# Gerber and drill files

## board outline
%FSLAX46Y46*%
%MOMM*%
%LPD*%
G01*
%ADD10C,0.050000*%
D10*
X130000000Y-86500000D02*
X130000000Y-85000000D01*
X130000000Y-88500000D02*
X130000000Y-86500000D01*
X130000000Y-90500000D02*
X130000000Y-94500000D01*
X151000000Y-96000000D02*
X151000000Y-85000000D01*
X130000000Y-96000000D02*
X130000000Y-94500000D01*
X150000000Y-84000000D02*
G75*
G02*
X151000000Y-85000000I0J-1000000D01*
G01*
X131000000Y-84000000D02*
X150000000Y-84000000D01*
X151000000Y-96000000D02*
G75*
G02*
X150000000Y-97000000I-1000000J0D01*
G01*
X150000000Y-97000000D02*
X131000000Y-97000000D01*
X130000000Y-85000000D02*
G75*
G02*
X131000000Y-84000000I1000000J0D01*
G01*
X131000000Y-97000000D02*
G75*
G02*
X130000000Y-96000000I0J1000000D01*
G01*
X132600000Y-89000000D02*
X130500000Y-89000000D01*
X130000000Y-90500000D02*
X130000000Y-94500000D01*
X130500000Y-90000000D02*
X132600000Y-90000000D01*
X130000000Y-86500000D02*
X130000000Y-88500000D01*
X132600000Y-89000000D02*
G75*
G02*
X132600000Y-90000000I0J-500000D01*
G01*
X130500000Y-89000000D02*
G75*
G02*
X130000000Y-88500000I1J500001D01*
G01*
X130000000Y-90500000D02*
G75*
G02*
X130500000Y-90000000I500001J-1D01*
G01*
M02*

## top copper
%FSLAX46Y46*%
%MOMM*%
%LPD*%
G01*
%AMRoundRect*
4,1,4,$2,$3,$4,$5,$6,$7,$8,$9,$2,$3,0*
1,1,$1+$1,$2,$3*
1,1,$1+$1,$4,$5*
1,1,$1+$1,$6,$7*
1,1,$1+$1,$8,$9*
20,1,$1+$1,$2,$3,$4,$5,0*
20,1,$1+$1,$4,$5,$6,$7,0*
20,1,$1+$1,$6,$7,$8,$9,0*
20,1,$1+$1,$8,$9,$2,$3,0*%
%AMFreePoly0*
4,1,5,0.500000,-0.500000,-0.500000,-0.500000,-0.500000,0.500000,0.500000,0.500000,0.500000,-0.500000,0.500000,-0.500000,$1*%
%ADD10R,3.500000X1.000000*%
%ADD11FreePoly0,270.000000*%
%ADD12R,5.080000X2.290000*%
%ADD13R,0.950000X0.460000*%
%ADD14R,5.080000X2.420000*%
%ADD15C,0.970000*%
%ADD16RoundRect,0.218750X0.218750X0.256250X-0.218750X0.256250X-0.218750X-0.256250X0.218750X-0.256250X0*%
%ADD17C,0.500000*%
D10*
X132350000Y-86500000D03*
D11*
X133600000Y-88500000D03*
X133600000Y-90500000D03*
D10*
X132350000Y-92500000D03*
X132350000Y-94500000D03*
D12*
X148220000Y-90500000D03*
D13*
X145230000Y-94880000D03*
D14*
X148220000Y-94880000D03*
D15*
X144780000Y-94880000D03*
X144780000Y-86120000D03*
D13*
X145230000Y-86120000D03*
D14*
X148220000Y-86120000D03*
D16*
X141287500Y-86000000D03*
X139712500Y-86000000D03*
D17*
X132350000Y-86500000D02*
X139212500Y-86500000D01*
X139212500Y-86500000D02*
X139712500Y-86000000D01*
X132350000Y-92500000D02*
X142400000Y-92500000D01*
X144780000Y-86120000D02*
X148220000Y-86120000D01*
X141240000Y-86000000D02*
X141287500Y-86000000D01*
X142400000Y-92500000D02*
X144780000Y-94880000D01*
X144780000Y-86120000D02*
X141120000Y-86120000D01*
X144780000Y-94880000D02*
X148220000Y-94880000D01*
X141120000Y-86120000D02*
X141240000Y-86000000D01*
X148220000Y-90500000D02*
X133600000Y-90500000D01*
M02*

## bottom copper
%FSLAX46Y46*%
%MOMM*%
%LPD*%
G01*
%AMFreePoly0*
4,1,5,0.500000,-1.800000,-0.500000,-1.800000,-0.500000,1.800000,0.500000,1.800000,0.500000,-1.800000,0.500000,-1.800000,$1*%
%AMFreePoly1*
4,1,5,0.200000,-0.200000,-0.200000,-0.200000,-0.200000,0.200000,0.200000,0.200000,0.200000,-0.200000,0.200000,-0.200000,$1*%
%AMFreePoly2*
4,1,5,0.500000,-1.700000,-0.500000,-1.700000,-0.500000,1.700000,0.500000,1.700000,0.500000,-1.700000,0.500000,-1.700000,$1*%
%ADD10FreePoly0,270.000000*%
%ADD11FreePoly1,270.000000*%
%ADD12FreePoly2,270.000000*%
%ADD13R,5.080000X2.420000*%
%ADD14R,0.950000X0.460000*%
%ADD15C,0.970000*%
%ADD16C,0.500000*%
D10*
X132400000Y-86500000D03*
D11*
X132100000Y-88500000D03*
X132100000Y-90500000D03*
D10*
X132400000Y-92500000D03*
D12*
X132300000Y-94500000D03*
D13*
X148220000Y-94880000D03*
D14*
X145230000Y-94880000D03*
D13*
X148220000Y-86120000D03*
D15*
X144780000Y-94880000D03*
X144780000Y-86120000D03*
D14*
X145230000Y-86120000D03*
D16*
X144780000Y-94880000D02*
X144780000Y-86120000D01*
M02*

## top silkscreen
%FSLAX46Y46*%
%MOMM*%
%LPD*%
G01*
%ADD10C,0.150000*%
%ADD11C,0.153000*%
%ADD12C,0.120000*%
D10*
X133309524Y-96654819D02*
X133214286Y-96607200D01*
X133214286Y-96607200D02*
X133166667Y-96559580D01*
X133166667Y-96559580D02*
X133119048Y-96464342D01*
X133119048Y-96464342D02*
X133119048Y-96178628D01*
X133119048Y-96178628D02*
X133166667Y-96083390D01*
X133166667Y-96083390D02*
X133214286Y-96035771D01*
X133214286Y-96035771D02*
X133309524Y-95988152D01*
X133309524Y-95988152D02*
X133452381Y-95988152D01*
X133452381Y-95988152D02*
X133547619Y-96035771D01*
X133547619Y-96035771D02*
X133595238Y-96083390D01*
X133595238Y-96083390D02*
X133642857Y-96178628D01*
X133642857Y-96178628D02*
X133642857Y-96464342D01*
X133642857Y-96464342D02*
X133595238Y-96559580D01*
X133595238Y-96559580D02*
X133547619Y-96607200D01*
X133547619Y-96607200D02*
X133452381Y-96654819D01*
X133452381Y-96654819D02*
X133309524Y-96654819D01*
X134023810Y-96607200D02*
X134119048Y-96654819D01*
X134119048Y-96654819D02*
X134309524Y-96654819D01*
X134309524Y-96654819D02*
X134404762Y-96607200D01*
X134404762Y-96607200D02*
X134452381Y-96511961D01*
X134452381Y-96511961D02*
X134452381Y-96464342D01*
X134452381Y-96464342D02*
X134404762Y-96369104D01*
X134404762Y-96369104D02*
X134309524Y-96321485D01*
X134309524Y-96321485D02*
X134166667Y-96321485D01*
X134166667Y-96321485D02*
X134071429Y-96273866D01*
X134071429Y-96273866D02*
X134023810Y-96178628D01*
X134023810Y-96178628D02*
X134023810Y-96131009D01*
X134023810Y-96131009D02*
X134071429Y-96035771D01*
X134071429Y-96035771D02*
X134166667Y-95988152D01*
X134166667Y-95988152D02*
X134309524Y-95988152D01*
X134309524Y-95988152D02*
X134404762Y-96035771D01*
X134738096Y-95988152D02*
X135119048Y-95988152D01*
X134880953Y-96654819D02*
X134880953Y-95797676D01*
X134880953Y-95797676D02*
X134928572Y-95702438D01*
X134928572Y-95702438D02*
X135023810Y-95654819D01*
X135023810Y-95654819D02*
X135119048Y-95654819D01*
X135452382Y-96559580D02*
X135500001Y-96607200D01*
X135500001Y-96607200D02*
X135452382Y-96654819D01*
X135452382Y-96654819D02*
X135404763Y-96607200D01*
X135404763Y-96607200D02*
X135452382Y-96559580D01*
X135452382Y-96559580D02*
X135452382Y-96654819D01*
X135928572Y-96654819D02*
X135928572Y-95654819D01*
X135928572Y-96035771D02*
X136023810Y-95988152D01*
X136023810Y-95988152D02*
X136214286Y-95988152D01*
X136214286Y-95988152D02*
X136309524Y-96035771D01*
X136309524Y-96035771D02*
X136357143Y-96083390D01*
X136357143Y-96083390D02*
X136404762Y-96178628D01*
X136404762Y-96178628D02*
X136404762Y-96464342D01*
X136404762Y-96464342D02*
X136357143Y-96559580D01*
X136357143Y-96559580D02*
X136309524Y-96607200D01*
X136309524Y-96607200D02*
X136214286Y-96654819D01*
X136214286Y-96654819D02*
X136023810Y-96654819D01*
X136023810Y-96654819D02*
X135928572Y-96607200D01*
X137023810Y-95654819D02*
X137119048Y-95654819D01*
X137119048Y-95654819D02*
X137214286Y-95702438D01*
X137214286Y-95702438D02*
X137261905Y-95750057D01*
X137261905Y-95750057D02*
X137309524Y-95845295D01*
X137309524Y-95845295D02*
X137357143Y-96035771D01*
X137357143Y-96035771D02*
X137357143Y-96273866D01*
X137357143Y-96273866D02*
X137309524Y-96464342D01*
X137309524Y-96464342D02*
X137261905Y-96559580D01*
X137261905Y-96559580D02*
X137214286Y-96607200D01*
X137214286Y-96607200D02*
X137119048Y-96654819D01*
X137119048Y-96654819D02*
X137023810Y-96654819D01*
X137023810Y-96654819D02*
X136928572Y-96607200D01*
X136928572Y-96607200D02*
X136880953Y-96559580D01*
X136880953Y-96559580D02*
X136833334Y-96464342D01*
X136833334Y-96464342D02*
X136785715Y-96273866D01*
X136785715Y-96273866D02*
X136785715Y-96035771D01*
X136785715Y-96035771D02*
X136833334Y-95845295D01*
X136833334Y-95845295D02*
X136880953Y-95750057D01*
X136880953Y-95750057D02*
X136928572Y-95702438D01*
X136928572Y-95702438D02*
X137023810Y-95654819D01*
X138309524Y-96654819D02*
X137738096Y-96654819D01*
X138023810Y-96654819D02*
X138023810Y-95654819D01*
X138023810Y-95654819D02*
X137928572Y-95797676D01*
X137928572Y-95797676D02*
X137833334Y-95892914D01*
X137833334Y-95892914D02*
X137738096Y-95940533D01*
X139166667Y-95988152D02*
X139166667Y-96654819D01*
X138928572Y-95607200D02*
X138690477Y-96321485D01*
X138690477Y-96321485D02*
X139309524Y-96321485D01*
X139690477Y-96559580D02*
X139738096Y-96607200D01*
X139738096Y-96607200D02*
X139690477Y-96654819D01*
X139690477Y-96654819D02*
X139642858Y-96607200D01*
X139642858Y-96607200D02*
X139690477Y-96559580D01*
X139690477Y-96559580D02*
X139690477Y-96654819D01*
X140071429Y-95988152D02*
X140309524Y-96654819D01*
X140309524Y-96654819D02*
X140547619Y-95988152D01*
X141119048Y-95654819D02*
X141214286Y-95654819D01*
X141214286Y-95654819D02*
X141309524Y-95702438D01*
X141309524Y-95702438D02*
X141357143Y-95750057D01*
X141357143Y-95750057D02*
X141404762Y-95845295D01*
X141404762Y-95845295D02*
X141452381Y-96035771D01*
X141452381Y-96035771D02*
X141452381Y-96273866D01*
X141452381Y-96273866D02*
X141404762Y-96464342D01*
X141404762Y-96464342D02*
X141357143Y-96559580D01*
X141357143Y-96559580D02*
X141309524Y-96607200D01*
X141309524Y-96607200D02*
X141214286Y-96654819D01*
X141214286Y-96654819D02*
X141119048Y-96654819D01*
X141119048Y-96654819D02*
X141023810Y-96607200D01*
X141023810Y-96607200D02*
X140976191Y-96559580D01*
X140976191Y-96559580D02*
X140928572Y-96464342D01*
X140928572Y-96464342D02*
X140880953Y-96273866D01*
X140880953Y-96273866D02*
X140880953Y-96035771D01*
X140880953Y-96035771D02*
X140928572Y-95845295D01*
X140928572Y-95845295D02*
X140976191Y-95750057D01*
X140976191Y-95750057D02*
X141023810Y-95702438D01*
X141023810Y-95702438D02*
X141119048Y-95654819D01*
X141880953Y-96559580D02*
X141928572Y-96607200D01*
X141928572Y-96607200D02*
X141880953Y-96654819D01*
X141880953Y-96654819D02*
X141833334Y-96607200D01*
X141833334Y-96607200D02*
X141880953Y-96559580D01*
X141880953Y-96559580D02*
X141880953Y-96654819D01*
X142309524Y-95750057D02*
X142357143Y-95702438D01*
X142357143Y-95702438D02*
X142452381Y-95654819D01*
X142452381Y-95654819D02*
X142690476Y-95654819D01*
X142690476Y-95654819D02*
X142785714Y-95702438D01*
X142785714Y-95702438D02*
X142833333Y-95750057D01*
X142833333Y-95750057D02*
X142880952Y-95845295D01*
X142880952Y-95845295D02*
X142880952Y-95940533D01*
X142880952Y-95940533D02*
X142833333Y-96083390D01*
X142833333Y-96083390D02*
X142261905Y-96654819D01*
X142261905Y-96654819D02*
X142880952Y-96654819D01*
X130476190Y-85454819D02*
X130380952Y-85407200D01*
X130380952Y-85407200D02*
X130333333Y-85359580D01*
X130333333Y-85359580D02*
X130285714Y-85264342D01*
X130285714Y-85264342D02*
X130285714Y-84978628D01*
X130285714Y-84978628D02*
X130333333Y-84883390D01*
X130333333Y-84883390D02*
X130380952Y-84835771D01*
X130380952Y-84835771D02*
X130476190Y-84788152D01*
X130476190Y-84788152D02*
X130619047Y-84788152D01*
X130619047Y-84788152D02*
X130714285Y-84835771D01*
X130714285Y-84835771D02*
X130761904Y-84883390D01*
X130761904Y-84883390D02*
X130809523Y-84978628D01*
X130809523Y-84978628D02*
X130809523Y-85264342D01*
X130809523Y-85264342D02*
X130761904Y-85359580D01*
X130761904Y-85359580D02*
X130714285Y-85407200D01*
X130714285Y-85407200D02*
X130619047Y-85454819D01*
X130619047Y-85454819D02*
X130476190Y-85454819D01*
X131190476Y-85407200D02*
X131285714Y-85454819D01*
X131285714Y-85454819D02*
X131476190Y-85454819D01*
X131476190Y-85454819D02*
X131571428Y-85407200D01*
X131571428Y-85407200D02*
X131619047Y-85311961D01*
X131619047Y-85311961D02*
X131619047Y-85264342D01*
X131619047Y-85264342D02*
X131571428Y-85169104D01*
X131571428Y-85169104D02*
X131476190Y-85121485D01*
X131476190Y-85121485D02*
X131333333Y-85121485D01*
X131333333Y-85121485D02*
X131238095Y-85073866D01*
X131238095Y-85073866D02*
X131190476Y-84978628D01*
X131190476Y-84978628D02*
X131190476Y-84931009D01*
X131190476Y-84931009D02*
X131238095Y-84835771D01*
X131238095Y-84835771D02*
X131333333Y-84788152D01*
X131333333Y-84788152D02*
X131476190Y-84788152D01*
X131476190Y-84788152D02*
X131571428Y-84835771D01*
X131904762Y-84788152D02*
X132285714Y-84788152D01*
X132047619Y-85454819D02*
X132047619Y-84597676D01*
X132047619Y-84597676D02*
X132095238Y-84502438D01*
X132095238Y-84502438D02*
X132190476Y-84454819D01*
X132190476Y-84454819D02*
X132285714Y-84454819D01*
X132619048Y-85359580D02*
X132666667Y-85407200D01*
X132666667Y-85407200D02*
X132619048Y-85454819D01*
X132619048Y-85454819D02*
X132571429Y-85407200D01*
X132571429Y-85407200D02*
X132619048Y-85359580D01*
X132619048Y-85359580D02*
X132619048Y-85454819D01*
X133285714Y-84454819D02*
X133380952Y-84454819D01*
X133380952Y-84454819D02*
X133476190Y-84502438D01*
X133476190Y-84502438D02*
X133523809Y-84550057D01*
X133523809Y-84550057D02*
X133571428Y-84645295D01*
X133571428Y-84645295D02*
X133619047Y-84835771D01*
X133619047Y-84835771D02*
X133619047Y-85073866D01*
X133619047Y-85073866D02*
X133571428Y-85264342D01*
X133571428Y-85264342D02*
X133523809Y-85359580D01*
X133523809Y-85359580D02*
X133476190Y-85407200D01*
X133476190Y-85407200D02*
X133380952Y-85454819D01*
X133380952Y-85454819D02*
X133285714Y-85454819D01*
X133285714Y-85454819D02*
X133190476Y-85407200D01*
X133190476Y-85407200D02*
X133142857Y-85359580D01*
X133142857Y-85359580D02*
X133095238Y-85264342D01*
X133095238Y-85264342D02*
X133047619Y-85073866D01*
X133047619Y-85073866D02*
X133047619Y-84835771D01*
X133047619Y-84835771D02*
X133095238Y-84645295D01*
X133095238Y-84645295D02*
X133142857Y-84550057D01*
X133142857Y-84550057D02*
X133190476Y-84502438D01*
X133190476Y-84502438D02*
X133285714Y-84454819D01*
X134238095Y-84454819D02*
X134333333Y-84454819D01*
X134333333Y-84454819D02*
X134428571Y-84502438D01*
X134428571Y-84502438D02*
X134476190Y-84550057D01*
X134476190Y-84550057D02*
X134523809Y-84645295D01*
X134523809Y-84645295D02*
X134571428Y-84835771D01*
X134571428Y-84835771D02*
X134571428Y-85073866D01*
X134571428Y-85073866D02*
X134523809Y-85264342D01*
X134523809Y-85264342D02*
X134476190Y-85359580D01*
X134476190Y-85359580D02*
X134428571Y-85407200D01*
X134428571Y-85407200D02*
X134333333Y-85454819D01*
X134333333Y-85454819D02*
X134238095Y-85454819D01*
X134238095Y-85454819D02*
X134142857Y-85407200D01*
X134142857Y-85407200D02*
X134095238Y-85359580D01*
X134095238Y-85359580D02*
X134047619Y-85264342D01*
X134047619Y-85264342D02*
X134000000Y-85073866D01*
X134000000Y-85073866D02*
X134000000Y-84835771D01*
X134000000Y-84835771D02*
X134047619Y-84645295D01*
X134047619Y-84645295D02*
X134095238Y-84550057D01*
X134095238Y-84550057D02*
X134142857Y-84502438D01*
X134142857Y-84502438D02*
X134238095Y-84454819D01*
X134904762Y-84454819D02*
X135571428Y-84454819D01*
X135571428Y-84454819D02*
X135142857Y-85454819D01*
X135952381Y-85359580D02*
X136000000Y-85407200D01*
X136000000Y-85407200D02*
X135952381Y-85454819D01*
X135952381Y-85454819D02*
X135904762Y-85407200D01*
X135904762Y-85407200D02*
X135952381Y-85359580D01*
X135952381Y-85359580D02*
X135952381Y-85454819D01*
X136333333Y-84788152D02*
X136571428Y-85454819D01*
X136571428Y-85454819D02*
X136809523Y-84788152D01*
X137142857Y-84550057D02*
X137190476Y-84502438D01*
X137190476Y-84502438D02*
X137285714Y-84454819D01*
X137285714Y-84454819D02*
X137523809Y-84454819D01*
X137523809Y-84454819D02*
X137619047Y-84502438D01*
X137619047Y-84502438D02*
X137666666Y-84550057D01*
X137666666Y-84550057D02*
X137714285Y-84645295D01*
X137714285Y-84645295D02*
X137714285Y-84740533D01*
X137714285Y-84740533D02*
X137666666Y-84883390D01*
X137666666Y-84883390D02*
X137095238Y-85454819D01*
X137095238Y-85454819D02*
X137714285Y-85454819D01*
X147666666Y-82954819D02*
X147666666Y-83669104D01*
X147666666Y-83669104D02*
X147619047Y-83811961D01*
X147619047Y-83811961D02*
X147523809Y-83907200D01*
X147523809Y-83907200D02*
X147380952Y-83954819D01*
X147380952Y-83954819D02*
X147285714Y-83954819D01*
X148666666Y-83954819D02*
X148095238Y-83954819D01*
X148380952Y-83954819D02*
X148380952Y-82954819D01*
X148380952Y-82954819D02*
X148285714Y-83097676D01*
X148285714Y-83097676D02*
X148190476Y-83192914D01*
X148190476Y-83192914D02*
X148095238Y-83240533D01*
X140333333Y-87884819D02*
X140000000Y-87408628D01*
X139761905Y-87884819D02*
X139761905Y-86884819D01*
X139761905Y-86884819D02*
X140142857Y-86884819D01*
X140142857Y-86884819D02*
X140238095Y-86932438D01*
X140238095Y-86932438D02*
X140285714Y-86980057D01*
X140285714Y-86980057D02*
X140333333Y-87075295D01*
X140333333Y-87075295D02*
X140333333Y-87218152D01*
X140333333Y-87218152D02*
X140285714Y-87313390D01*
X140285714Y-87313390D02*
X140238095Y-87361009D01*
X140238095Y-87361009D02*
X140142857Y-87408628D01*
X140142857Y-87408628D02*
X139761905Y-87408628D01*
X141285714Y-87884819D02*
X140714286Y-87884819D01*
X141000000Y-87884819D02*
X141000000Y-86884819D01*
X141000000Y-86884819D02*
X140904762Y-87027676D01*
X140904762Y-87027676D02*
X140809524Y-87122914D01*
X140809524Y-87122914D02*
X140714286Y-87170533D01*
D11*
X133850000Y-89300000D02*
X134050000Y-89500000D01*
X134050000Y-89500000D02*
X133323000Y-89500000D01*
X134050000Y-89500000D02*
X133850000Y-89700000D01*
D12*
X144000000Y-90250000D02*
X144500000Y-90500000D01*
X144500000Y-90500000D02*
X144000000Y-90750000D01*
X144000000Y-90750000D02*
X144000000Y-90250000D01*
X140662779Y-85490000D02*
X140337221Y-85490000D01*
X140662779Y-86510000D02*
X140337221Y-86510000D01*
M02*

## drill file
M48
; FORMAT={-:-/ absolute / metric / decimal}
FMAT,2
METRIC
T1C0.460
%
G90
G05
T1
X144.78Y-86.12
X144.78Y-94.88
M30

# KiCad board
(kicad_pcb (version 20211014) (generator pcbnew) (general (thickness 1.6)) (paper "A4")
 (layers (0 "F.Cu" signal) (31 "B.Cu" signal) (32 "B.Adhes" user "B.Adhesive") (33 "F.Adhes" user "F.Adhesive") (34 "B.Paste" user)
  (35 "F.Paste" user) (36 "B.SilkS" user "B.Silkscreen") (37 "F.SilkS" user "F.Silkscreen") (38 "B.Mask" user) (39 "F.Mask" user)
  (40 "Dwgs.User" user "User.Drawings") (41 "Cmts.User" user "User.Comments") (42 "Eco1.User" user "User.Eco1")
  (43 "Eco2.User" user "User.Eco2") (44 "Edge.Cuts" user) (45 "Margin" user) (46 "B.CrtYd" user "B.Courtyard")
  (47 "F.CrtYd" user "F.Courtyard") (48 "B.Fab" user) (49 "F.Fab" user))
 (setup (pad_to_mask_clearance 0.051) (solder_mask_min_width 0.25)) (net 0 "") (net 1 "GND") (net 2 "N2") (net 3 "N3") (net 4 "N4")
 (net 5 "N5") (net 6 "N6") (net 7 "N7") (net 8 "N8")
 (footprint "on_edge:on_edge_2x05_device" (layer "F.Cu") (at 130 90.5 -90)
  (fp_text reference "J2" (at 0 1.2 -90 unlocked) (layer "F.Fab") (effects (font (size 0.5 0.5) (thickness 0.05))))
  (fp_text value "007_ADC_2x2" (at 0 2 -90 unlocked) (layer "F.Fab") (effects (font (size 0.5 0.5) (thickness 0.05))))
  (fp_line (start -1.2 -3.85) (end -1 -4.05) (layer "F.SilkS") (width 0.153))
  (fp_line (start -1 -4.05) (end -1 -3.323) (layer "F.SilkS") (width 0.153))
  (fp_line (start -1 -4.05) (end -0.8 -3.85) (layer "F.SilkS") (width 0.153))
  (fp_line (start -1.5 -2.6) (end -1.5 -0.5) (layer "Edge.Cuts") (width 0.05))
  (fp_line (start 0 0) (end 4 0) (layer "Edge.Cuts") (width 0.05))
  (fp_line (start -0.5 -0.5) (end -0.5 -2.6) (layer "Edge.Cuts") (width 0.05))
  (fp_line (start -4 0) (end -2 0) (layer "Edge.Cuts") (width 0.05))
  (fp_arc (start -1.5 -2.6) (mid -1 -3.1) (end -0.5 -2.6) (layer "Edge.Cuts") (width 0.05))
  (fp_arc (start -1.5 -0.5) (mid -1.646447 -0.146447) (end -2 0) (layer "Edge.Cuts") (width 0.05))
  (fp_arc (start 0 0) (mid -0.353553 -0.146447) (end -0.5 -0.5) (layer "Edge.Cuts") (width 0.05))
  (pad "1" smd rect locked (at -4 -2.35 90) (size 1 3.5) (layers "F.Cu" "F.Mask") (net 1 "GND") (zone_connect 0))
  (pad "2" smd custom locked (at -2 -3.6 270) (size 1 1) (layers "F.Cu" "F.Mask") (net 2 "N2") (zone_connect 0)
   (options (clearance outline) (anchor rect)) (primitives))
  (pad "3" smd custom locked (at 0 -3.6 270) (size 1 1) (layers "F.Cu" "F.Mask") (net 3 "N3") (zone_connect 0)
   (options (clearance outline) (anchor rect)) (primitives))
  (pad "4" smd rect locked (at 2 -2.35 90) (size 1 3.5) (layers "F.Cu" "F.Mask") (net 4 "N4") (zone_connect 0))
  (pad "5" smd rect locked (at 4 -2.35 90) (size 1 3.5) (layers "F.Cu" "F.Mask") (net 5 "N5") (zone_connect 0))
  (pad "6" smd custom locked (at -4 -2.4 270) (size 1 3.6) (layers "B.Cu" "B.Mask") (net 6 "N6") (zone_connect 0)
   (options (clearance outline) (anchor rect)) (primitives))
  (pad "7" smd custom locked (at -2 -2.1 270) (size 0.4 0.4) (layers "B.Cu" "B.Mask") (zone_connect 0)
   (options (clearance outline) (anchor rect)) (primitives))
  (pad "8" smd custom locked (at 0 -2.1 270) (size 0.4 0.4) (layers "B.Cu" "B.Mask") (zone_connect 0)
   (options (clearance outline) (anchor rect)) (primitives))
  (pad "9" smd custom locked (at 2 -2.4 270) (size 1 3.6) (layers "B.Cu" "B.Mask") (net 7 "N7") (zone_connect 0)
   (options (clearance outline) (anchor rect)) (primitives))
  (pad "10" smd custom locked (at 4 -2.3 270) (size 1 3.4) (layers "B.Cu" "B.Mask") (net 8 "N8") (zone_connect 0)
   (options (clearance outline) (anchor rect)) (primitives)))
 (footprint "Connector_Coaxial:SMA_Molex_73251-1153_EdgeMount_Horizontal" (layer "F.Cu") (at 146.5 90.5 180)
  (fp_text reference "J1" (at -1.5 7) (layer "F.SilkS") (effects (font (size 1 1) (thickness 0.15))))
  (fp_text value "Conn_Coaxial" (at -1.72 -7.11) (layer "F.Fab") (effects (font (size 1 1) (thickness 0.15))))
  (fp_line (start 2.5 0.25) (end 2 0) (layer "F.SilkS") (width 0.12))
  (fp_line (start 2 0) (end 2.5 -0.25) (layer "F.SilkS") (width 0.12))
  (fp_line (start 2.5 -0.25) (end 2.5 0.25) (layer "F.SilkS") (width 0.12))
  (pad "1" smd rect locked (at -1.72 0 180) (size 5.08 2.29) (layers "F.Cu" "F.Paste" "F.Mask") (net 3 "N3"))
  (pad "2" smd rect locked (at 1.27 -4.38 180) (size 0.95 0.46) (layers "F.Cu") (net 4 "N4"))
  (pad "2" smd rect locked (at -1.72 -4.38 180) (size 5.08 2.42) (layers "B.Cu" "B.Paste" "B.Mask") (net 4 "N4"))
  (pad "2" smd rect locked (at -1.72 -4.38 180) (size 5.08 2.42) (layers "F.Cu" "F.Paste" "F.Mask") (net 4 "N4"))
  (pad "2" smd rect locked (at 1.27 -4.38 180) (size 0.95 0.46) (layers "B.Cu") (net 4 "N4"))
  (pad "2" smd rect locked (at -1.72 4.38 180) (size 5.08 2.42) (layers "B.Cu" "B.Paste" "B.Mask") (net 4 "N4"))
  (pad "2" thru_hole circle locked (at 1.72 -4.38 180) (size 0.97 0.97) (drill 0.46) (layers *.Cu) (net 4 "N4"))
  (pad "2" thru_hole circle locked (at 1.72 4.38 180) (size 0.97 0.97) (drill 0.46) (layers *.Cu) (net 4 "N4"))
  (pad "2" smd rect locked (at 1.27 4.38 180) (size 0.95 0.46) (layers "B.Cu") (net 4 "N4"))
  (pad "2" smd rect locked (at 1.27 4.38 180) (size 0.95 0.46) (layers "F.Cu") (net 4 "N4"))
  (pad "2" smd rect locked (at -1.72 4.38 180) (size 5.08 2.42) (layers "F.Cu" "F.Paste" "F.Mask") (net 4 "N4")))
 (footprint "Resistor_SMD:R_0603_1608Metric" (layer "F.Cu") (at 140.5 86 180)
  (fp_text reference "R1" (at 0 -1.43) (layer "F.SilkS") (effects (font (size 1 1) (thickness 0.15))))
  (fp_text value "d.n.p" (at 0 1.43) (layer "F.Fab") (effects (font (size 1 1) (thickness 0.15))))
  (fp_line (start -0.162779 0.51) (end 0.162779 0.51) (layer "F.SilkS") (width 0.12))
  (fp_line (start -0.162779 -0.51) (end 0.162779 -0.51) (layer "F.SilkS") (width 0.12))
  (pad "1" smd roundrect locked (at -0.7875 0 180) (size 0.875 0.95) (layers "F.Cu" "F.Paste" "F.Mask") (roundrect_rratio 0.25) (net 4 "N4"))
  (pad "2" smd roundrect locked (at 0.7875 0 180) (size 0.875 0.95) (layers "F.Cu" "F.Paste" "F.Mask") (roundrect_rratio 0.25) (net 1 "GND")))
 (gr_line (start 130 86.5) (end 130 85) (layer "Edge.Cuts") (width 0.05))
 (gr_line (start 130 88.5) (end 130 86.5) (layer "Edge.Cuts") (width 0.05))
 (gr_line (start 130 90.5) (end 130 94.5) (layer "Edge.Cuts") (width 0.05))
 (gr_line (start 151 96) (end 151 85) (layer "Edge.Cuts") (width 0.05))
 (gr_line (start 130 96) (end 130 94.5) (layer "Edge.Cuts") (width 0.05))
 (gr_arc (start 150 84) (mid 150.707107 84.292893) (end 151 85) (layer "Edge.Cuts") (width 0.05))
 (gr_line (start 131 84) (end 150 84) (layer "Edge.Cuts") (width 0.05))
 (gr_arc (start 151 96) (mid 150.707107 96.707107) (end 150 97) (layer "Edge.Cuts") (width 0.05))
 (gr_line (start 150 97) (end 131 97) (layer "Edge.Cuts") (width 0.05))
 (gr_arc (start 130 85) (mid 130.292893 84.292893) (end 131 84) (layer "Edge.Cuts") (width 0.05))
 (gr_arc (start 131 97) (mid 130.292893 96.707107) (end 130 96) (layer "Edge.Cuts") (width 0.05))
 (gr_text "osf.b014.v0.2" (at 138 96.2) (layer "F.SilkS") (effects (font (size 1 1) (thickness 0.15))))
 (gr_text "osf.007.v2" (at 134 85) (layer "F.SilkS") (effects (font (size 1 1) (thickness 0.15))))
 (segment (start 132.35 86.5) (end 139.2125 86.5) (width 0.5) (layer "F.Cu") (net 1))
 (segment (start 139.2125 86.5) (end 139.7125 86) (width 0.5) (layer "F.Cu") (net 1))
 (segment (start 132.35 92.5) (end 142.4 92.5) (width 0.5) (layer "F.Cu") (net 4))
 (segment (start 144.78 86.12) (end 148.22 86.12) (width 0.5) (layer "F.Cu") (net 4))
 (segment (start 141.24 86) (end 141.2875 86) (width 0.5) (layer "F.Cu") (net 4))
 (segment (start 142.4 92.5) (end 144.78 94.88) (width 0.5) (layer "F.Cu") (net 4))
 (segment (start 144.78 86.12) (end 141.12 86.12) (width 0.5) (layer "F.Cu") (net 4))
 (segment (start 144.78 94.88) (end 148.22 94.88) (width 0.5) (layer "F.Cu") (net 4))
 (segment (start 141.12 86.12) (end 141.24 86) (width 0.5) (layer "F.Cu") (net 4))
 (segment (start 144.78 94.88) (end 144.78 86.12) (width 0.5) (layer "B.Cu") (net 4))
 (segment (start 148.22 90.5) (end 133.6 90.5) (width 0.5) (layer "F.Cu") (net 3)))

